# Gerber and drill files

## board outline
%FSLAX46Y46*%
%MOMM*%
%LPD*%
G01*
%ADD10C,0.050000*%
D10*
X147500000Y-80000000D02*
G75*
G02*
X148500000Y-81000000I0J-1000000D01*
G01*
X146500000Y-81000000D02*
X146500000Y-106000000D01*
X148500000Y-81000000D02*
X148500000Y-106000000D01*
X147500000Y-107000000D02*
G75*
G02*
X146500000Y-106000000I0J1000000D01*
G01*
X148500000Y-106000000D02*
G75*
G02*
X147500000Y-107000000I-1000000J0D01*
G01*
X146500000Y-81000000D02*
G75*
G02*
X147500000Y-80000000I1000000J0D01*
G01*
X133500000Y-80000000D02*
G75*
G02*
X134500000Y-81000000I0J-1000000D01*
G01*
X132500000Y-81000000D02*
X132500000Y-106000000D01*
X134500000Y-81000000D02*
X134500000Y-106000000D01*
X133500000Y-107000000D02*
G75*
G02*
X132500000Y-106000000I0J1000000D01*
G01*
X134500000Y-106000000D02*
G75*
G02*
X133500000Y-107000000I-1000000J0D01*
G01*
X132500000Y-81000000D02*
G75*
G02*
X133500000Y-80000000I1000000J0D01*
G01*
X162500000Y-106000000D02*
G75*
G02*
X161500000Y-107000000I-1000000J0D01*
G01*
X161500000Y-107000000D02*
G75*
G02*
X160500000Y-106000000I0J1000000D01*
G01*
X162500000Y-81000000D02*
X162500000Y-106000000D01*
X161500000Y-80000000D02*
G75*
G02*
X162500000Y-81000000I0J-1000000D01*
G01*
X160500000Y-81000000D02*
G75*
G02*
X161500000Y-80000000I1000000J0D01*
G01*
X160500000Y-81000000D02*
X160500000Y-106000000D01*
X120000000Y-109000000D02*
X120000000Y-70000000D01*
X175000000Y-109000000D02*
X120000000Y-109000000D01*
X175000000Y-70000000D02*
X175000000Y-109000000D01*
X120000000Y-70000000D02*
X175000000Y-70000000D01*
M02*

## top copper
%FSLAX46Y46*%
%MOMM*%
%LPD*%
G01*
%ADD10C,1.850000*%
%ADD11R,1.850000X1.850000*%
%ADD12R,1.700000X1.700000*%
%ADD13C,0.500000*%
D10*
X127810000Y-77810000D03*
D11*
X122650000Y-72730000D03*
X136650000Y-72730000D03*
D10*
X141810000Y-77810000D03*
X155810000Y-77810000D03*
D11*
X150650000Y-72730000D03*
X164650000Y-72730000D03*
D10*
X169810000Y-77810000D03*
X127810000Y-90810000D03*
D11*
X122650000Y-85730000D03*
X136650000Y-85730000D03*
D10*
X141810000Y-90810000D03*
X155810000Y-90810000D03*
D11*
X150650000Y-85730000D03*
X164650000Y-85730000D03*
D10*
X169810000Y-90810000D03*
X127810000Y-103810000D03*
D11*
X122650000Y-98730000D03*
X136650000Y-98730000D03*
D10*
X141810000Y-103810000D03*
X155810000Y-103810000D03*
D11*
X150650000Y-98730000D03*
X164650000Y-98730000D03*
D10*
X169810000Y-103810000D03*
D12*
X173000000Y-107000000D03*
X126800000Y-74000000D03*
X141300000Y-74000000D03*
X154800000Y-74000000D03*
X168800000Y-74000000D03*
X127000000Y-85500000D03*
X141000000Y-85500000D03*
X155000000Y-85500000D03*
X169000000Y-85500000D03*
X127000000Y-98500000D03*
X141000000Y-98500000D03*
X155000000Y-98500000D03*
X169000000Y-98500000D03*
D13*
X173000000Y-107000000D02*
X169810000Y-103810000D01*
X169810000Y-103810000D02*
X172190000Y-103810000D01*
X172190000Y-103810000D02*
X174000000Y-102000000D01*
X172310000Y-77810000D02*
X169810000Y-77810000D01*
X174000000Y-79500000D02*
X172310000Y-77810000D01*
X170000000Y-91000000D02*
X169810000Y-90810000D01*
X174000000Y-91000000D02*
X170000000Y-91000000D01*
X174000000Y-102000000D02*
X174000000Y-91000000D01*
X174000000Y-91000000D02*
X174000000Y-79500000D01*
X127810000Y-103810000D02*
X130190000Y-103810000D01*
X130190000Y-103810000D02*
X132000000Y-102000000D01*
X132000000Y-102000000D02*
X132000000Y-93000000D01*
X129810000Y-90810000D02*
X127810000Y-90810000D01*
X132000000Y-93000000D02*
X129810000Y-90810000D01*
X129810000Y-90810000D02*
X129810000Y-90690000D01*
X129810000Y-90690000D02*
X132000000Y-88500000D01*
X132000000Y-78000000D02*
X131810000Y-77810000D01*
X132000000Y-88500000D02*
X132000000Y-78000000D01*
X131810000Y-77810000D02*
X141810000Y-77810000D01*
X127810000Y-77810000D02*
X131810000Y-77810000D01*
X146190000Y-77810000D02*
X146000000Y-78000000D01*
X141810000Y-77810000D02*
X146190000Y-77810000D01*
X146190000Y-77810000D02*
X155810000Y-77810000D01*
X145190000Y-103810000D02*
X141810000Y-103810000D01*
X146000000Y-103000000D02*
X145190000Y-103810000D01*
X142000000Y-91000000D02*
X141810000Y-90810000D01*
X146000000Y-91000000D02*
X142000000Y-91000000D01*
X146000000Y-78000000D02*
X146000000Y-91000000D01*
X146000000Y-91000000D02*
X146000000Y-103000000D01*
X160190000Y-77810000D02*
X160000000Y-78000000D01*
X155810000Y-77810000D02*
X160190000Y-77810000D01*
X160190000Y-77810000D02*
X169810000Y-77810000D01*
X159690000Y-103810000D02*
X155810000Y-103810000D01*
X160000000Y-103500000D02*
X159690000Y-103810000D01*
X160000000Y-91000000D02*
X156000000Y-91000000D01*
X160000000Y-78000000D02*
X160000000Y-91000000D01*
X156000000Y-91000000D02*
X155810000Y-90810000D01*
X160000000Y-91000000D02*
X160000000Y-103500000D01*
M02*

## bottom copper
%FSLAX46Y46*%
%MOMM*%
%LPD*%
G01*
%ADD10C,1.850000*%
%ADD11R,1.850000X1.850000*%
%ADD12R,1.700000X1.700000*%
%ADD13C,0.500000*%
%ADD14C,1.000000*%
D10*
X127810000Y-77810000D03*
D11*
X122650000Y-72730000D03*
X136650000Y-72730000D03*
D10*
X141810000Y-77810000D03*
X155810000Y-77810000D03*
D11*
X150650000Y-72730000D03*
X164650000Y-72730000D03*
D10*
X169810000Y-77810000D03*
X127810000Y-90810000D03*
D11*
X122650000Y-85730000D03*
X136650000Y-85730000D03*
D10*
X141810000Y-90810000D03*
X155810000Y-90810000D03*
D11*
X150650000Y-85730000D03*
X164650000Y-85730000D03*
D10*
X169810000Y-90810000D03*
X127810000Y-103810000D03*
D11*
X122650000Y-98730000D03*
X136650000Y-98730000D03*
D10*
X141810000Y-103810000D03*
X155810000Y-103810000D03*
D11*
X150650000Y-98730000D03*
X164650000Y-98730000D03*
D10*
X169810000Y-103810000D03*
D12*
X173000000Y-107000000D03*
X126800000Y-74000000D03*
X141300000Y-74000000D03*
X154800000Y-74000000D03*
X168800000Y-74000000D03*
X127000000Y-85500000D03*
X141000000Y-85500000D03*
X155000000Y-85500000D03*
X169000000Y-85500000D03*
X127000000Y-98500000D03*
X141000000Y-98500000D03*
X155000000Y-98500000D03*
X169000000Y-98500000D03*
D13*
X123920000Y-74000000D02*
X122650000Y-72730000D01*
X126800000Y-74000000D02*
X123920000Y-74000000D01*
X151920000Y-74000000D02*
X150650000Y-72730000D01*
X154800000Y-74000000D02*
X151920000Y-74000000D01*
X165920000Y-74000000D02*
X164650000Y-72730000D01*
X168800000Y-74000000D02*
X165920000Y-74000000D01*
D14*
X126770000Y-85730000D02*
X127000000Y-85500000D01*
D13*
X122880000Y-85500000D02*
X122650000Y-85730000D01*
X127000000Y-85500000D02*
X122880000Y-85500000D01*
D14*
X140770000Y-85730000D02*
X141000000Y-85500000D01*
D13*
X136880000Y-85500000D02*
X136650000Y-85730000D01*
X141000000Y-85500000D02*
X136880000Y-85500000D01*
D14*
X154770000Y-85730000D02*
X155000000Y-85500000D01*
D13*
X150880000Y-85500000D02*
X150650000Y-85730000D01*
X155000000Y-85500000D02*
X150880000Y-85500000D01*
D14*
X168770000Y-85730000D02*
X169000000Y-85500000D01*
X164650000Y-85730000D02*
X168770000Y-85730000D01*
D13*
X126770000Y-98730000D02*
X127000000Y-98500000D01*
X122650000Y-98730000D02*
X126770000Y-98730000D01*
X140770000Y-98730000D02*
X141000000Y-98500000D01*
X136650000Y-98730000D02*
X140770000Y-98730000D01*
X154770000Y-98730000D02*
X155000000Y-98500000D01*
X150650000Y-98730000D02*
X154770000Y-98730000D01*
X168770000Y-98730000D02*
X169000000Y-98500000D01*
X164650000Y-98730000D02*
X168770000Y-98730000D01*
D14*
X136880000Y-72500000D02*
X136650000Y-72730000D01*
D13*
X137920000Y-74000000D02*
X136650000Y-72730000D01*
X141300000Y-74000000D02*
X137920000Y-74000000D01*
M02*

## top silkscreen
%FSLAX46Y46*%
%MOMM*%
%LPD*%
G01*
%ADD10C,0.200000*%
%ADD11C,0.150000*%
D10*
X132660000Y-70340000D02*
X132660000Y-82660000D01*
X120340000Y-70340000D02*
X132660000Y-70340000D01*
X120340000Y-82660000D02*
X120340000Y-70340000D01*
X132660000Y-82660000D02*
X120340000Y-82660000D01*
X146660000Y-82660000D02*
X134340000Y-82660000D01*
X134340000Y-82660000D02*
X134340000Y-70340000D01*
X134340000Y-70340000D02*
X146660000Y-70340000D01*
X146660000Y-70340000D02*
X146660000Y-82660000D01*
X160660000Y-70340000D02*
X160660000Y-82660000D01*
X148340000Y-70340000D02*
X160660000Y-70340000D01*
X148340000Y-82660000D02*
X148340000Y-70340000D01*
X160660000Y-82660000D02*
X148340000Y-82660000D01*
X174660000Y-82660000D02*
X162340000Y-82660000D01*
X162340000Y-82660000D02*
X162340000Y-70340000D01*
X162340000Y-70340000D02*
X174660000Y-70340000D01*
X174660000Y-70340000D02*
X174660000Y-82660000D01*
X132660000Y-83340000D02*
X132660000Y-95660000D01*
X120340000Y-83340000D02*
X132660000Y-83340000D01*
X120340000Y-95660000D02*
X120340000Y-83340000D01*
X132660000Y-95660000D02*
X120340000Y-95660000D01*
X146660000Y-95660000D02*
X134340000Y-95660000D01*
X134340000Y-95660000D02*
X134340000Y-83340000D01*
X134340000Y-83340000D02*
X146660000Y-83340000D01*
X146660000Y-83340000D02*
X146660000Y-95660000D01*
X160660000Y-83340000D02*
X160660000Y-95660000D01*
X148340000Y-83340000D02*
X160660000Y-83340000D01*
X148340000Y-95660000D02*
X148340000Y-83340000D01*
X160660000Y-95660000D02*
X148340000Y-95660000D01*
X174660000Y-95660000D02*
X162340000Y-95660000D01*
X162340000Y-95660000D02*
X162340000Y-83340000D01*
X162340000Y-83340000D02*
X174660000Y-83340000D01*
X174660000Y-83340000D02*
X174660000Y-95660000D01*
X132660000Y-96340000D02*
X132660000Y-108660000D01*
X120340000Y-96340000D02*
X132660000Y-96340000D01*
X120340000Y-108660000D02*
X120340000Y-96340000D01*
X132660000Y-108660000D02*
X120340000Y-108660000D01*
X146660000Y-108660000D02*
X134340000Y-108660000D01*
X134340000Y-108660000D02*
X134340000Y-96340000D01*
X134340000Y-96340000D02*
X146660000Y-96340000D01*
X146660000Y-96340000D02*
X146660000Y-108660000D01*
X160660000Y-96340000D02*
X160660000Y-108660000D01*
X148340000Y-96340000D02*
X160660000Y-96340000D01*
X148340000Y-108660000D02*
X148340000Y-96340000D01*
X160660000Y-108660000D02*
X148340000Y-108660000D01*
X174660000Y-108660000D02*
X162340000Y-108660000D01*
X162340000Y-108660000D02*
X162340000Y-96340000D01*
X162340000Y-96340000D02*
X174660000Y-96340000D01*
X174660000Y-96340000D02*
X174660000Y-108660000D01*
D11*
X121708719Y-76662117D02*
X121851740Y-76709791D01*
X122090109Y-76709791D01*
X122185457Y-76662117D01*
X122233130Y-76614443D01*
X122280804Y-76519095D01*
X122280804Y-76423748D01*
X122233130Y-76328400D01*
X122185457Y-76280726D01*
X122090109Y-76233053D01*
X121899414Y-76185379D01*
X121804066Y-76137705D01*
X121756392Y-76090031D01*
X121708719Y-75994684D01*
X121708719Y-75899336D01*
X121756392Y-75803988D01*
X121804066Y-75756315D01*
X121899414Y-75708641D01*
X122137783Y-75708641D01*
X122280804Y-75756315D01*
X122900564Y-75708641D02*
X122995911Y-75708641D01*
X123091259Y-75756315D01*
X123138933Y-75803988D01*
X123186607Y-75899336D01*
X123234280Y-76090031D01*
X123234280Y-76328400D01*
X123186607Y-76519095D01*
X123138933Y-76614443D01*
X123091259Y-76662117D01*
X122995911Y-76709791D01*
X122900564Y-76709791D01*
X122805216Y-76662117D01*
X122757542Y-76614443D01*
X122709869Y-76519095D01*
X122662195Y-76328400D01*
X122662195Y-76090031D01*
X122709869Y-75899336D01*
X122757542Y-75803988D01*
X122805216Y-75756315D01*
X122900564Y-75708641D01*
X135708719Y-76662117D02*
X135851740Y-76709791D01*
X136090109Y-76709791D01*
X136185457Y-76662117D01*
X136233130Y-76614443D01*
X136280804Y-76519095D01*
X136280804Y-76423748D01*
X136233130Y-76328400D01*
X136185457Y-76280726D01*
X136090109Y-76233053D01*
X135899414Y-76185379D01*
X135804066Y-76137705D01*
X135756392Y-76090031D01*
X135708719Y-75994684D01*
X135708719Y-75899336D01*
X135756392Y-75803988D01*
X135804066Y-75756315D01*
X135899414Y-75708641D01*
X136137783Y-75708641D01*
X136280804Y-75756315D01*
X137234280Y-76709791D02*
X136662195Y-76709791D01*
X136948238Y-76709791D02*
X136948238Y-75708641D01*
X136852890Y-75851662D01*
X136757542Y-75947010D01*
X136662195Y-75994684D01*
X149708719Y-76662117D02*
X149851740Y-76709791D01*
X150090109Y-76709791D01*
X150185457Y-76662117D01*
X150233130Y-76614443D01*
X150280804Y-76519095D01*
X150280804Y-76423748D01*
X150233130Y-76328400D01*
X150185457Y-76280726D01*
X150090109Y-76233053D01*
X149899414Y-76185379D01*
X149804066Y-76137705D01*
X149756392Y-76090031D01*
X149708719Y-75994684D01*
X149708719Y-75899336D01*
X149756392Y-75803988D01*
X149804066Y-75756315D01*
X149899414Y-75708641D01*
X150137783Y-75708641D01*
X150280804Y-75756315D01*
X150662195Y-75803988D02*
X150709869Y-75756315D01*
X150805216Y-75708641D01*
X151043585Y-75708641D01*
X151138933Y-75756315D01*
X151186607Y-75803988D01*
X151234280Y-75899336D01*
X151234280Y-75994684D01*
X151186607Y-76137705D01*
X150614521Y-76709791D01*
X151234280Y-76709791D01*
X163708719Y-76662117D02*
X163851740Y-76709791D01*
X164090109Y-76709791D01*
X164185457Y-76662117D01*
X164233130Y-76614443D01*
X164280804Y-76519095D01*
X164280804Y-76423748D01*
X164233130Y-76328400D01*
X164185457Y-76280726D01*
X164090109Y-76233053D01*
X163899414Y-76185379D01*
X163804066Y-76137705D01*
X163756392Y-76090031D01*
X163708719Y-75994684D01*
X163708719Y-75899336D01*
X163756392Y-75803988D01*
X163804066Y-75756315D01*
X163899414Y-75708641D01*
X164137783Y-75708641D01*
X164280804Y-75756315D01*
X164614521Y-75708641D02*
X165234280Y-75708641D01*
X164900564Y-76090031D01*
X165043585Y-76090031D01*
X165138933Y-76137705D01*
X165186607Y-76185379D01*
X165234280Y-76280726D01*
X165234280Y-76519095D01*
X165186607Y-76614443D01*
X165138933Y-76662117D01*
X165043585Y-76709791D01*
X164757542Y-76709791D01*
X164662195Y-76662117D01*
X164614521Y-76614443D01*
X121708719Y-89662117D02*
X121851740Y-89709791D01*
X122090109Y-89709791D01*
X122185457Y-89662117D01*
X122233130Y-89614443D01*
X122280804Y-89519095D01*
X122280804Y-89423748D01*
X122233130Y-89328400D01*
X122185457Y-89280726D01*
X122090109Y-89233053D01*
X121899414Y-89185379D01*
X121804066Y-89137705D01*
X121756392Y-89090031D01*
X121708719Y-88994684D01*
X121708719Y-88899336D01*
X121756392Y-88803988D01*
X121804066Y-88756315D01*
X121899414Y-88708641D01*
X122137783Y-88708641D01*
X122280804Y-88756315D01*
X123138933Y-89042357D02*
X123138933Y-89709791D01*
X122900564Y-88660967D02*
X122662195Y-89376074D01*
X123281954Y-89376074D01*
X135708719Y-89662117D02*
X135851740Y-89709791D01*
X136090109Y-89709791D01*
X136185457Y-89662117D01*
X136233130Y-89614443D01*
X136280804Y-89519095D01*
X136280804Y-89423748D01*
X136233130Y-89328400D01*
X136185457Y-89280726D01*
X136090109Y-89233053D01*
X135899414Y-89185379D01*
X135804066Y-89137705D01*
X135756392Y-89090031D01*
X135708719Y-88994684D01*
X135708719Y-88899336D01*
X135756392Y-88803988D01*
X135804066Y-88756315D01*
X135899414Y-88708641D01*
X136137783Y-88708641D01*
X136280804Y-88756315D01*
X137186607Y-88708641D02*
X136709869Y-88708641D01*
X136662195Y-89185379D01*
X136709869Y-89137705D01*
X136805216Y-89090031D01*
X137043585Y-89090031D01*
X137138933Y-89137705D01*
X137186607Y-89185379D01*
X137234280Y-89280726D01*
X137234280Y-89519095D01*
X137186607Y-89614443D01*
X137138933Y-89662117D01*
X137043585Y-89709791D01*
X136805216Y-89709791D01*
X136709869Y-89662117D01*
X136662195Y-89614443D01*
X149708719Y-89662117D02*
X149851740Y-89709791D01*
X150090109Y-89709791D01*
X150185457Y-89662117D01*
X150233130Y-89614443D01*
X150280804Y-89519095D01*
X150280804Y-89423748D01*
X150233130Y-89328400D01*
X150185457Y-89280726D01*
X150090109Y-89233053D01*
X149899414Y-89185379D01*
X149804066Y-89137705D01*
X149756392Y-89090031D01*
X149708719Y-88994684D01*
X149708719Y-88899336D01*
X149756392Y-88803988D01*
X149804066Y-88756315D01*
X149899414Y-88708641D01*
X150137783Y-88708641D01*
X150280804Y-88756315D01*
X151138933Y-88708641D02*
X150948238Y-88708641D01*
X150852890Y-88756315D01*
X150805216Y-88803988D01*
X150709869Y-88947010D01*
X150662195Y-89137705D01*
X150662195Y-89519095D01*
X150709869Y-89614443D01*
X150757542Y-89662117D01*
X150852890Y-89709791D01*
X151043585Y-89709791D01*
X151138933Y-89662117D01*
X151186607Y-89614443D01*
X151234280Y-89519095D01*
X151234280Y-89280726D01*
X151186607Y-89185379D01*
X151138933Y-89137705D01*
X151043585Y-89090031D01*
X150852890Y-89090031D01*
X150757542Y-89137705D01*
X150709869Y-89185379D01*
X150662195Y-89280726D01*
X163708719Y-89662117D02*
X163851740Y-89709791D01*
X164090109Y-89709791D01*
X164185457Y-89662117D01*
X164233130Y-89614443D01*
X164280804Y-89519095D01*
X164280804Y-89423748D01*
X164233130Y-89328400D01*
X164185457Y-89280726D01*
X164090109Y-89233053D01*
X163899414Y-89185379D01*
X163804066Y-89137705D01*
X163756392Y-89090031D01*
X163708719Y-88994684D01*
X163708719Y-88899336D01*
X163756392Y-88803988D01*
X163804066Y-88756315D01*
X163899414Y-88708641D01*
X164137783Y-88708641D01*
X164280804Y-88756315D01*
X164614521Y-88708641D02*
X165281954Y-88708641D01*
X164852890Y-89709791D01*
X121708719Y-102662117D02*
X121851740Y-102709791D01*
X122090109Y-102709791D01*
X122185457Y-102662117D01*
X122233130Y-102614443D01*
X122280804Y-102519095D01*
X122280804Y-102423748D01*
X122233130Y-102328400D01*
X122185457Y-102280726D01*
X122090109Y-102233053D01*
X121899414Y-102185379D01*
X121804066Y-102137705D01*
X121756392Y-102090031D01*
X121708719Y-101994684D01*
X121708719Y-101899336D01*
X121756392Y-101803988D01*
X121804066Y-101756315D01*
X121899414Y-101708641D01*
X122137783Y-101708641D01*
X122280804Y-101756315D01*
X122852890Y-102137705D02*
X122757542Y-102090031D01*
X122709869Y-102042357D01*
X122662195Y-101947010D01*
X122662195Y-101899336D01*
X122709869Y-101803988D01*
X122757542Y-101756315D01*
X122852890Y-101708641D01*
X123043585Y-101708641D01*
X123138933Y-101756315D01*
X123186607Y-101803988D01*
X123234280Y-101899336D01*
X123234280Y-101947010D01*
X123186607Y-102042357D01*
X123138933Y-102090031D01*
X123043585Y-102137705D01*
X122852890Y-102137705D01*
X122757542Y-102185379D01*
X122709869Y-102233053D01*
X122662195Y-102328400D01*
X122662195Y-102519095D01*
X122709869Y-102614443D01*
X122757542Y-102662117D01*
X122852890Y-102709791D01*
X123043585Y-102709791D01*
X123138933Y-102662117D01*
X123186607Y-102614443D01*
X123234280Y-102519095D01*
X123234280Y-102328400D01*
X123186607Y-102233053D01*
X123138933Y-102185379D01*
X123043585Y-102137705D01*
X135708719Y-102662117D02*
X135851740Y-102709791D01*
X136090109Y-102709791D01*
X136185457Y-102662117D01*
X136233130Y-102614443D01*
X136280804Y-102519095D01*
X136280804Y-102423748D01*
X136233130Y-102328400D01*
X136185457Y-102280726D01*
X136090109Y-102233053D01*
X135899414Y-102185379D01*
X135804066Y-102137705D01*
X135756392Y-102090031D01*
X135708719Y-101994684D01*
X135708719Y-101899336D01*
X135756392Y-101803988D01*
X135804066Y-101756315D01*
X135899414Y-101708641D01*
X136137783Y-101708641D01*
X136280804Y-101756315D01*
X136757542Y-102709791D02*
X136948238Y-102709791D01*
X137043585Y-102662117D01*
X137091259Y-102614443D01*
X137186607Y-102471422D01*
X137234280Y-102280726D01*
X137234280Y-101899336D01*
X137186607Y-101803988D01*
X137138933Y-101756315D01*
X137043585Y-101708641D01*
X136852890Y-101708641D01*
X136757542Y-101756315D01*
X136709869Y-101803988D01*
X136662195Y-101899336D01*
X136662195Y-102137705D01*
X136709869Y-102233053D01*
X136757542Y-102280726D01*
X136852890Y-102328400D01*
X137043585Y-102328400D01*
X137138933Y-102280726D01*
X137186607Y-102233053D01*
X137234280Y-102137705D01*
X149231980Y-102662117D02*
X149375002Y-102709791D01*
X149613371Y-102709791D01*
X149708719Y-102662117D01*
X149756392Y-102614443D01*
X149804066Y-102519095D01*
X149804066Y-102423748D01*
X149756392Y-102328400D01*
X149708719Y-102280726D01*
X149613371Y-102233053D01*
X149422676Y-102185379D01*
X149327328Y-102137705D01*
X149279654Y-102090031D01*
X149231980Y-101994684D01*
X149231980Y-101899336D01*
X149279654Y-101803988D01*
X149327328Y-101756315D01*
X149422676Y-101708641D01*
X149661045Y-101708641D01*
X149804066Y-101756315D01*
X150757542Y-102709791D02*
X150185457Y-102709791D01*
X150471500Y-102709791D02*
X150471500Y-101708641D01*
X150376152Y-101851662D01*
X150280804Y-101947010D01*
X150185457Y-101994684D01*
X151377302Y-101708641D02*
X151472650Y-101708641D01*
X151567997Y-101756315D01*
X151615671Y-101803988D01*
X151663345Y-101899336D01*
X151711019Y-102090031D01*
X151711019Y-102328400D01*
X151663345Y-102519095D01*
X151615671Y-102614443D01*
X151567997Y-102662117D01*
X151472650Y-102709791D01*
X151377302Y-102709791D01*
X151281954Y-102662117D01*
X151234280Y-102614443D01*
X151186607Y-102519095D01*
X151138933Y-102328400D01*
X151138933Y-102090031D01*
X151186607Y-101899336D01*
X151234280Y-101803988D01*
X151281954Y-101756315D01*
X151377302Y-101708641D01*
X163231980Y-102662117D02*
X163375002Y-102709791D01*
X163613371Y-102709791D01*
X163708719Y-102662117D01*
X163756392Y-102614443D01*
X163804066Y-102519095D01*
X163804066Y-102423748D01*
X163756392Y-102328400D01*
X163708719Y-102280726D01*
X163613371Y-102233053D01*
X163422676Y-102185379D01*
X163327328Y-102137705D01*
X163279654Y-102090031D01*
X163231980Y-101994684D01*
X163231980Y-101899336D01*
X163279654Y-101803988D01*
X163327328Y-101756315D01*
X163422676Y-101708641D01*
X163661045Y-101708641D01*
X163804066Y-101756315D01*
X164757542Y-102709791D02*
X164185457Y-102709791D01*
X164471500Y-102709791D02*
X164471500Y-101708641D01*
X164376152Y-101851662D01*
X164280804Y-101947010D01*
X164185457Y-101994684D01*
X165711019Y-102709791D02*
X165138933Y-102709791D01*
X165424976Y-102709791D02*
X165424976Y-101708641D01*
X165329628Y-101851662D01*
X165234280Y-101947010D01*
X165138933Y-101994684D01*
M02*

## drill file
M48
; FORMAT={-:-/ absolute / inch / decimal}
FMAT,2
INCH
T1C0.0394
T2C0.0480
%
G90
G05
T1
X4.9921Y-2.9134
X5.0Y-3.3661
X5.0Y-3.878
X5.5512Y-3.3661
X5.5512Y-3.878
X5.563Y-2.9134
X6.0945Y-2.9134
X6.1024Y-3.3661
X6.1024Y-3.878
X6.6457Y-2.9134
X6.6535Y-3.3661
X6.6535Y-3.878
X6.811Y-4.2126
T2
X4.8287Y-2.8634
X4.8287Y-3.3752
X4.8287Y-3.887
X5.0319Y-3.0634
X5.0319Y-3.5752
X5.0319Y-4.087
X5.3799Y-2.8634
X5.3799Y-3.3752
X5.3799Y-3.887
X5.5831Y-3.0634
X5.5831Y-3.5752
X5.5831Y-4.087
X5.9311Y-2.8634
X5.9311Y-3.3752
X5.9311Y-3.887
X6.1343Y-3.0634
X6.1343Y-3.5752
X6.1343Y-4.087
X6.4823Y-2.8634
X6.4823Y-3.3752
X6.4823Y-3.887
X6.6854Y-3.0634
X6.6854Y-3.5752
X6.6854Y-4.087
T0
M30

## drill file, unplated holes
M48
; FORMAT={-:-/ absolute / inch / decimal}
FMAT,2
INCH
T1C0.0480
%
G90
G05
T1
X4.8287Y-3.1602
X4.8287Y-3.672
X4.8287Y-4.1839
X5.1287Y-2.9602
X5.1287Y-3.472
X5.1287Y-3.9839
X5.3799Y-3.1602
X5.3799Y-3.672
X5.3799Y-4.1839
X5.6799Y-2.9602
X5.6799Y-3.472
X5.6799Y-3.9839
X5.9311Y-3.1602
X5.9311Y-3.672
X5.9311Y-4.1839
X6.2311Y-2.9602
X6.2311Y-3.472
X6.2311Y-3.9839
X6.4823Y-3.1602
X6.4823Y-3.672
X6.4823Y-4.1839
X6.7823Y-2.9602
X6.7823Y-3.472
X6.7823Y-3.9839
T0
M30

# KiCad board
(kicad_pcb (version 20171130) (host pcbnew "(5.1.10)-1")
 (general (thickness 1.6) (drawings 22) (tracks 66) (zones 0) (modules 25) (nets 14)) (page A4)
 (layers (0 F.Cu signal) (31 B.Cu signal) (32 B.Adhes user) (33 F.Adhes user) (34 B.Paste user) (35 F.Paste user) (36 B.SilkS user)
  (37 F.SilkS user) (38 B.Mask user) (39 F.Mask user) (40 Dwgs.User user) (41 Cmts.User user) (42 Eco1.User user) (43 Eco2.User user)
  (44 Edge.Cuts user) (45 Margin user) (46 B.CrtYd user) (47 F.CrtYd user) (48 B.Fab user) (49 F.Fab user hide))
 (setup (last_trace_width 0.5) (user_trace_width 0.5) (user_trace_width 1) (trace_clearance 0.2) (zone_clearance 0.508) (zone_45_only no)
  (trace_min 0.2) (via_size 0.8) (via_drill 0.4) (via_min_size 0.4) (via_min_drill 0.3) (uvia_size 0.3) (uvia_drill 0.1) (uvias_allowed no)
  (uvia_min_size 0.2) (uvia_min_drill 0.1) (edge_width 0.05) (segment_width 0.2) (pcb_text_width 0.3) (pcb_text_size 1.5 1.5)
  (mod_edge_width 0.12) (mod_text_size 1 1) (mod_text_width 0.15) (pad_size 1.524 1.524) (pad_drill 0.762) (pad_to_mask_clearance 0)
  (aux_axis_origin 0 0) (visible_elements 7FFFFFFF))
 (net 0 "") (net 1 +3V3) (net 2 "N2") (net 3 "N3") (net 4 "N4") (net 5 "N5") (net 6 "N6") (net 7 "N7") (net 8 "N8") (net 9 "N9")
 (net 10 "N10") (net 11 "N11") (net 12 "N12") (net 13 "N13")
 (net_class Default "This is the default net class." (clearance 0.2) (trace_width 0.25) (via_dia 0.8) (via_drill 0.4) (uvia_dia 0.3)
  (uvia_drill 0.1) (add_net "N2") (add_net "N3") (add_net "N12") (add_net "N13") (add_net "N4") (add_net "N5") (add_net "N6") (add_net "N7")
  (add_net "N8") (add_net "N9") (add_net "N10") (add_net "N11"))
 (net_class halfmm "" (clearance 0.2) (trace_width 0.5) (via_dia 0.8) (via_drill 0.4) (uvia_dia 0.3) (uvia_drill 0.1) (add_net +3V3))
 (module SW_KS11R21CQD (layer F.Cu) (at 126.5 76.5)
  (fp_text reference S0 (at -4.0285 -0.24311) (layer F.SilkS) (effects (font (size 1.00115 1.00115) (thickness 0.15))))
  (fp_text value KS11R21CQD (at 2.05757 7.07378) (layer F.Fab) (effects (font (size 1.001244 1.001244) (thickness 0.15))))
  (fp_line (start 6.16 -6.16) (end 6.16 6.16) (layer F.SilkS) (width 0.2))
  (fp_line (start -6.16 -6.16) (end 6.16 -6.16) (layer F.SilkS) (width 0.2))
  (fp_line (start -6.16 6.16) (end -6.16 -6.16) (layer F.SilkS) (width 0.2))
  (fp_line (start 6.16 6.16) (end -6.16 6.16) (layer F.SilkS) (width 0.2))
  (pad None np_thru_hole circle (at -3.85 3.77) (size 1.22 1.22) (drill 1.22) (layers *.Cu *.Mask))
  (pad None np_thru_hole circle (at 3.77 -1.31) (size 1.22 1.22) (drill 1.22) (layers *.Cu *.Mask))
  (pad 3 thru_hole circle (at 1.31 1.31) (size 1.85 1.85) (drill 1.22) (layers *.Cu *.Mask) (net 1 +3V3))
  (pad 1 thru_hole rect (at -3.85 -3.77) (size 1.85 1.85) (drill 1.22) (layers *.Cu *.Mask) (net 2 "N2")))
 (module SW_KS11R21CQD (layer F.Cu) (at 140.5 76.5)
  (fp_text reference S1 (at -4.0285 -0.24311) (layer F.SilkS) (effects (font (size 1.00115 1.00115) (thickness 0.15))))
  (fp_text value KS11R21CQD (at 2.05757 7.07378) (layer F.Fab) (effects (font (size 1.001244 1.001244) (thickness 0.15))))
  (fp_line (start 6.16 6.16) (end -6.16 6.16) (layer F.SilkS) (width 0.2))
  (fp_line (start -6.16 6.16) (end -6.16 -6.16) (layer F.SilkS) (width 0.2))
  (fp_line (start -6.16 -6.16) (end 6.16 -6.16) (layer F.SilkS) (width 0.2))
  (fp_line (start 6.16 -6.16) (end 6.16 6.16) (layer F.SilkS) (width 0.2))
  (pad 1 thru_hole rect (at -3.85 -3.77) (size 1.85 1.85) (drill 1.22) (layers *.Cu *.Mask) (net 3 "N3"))
  (pad 3 thru_hole circle (at 1.31 1.31) (size 1.85 1.85) (drill 1.22) (layers *.Cu *.Mask) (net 1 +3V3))
  (pad None np_thru_hole circle (at 3.77 -1.31) (size 1.22 1.22) (drill 1.22) (layers *.Cu *.Mask))
  (pad None np_thru_hole circle (at -3.85 3.77) (size 1.22 1.22) (drill 1.22) (layers *.Cu *.Mask)))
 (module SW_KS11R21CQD (layer F.Cu) (at 154.5 76.5)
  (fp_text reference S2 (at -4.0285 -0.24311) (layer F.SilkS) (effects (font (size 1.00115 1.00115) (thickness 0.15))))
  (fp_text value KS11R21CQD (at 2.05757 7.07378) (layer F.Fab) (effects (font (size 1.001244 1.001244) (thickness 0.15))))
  (fp_line (start 6.16 -6.16) (end 6.16 6.16) (layer F.SilkS) (width 0.2))
  (fp_line (start -6.16 -6.16) (end 6.16 -6.16) (layer F.SilkS) (width 0.2))
  (fp_line (start -6.16 6.16) (end -6.16 -6.16) (layer F.SilkS) (width 0.2))
  (fp_line (start 6.16 6.16) (end -6.16 6.16) (layer F.SilkS) (width 0.2))
  (pad None np_thru_hole circle (at -3.85 3.77) (size 1.22 1.22) (drill 1.22) (layers *.Cu *.Mask))
  (pad None np_thru_hole circle (at 3.77 -1.31) (size 1.22 1.22) (drill 1.22) (layers *.Cu *.Mask))
  (pad 3 thru_hole circle (at 1.31 1.31) (size 1.85 1.85) (drill 1.22) (layers *.Cu *.Mask) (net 1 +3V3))
  (pad 1 thru_hole rect (at -3.85 -3.77) (size 1.85 1.85) (drill 1.22) (layers *.Cu *.Mask) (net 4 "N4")))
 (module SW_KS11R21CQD (layer F.Cu) (at 168.5 76.5)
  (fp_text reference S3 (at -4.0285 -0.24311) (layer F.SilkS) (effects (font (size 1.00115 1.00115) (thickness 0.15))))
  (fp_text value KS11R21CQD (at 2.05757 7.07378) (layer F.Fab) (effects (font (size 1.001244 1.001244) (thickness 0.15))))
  (fp_line (start 6.16 6.16) (end -6.16 6.16) (layer F.SilkS) (width 0.2))
  (fp_line (start -6.16 6.16) (end -6.16 -6.16) (layer F.SilkS) (width 0.2))
  (fp_line (start -6.16 -6.16) (end 6.16 -6.16) (layer F.SilkS) (width 0.2))
  (fp_line (start 6.16 -6.16) (end 6.16 6.16) (layer F.SilkS) (width 0.2))
  (pad 1 thru_hole rect (at -3.85 -3.77) (size 1.85 1.85) (drill 1.22) (layers *.Cu *.Mask) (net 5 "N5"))
  (pad 3 thru_hole circle (at 1.31 1.31) (size 1.85 1.85) (drill 1.22) (layers *.Cu *.Mask) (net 1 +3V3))
  (pad None np_thru_hole circle (at 3.77 -1.31) (size 1.22 1.22) (drill 1.22) (layers *.Cu *.Mask))
  (pad None np_thru_hole circle (at -3.85 3.77) (size 1.22 1.22) (drill 1.22) (layers *.Cu *.Mask)))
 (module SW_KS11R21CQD (layer F.Cu) (at 126.5 89.5)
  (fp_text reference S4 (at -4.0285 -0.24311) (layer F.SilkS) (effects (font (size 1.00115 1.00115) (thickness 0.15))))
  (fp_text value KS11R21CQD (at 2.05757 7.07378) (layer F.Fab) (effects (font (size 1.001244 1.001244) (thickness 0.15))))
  (fp_line (start 6.16 -6.16) (end 6.16 6.16) (layer F.SilkS) (width 0.2))
  (fp_line (start -6.16 -6.16) (end 6.16 -6.16) (layer F.SilkS) (width 0.2))
  (fp_line (start -6.16 6.16) (end -6.16 -6.16) (layer F.SilkS) (width 0.2))
  (fp_line (start 6.16 6.16) (end -6.16 6.16) (layer F.SilkS) (width 0.2))
  (pad None np_thru_hole circle (at -3.85 3.77) (size 1.22 1.22) (drill 1.22) (layers *.Cu *.Mask))
  (pad None np_thru_hole circle (at 3.77 -1.31) (size 1.22 1.22) (drill 1.22) (layers *.Cu *.Mask))
  (pad 3 thru_hole circle (at 1.31 1.31) (size 1.85 1.85) (drill 1.22) (layers *.Cu *.Mask) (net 1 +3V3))
  (pad 1 thru_hole rect (at -3.85 -3.77) (size 1.85 1.85) (drill 1.22) (layers *.Cu *.Mask) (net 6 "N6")))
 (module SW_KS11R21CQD (layer F.Cu) (at 140.5 89.5)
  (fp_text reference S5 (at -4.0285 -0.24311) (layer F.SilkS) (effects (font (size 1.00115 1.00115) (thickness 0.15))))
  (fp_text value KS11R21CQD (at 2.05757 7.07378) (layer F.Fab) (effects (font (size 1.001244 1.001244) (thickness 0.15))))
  (fp_line (start 6.16 6.16) (end -6.16 6.16) (layer F.SilkS) (width 0.2))
  (fp_line (start -6.16 6.16) (end -6.16 -6.16) (layer F.SilkS) (width 0.2))
  (fp_line (start -6.16 -6.16) (end 6.16 -6.16) (layer F.SilkS) (width 0.2))
  (fp_line (start 6.16 -6.16) (end 6.16 6.16) (layer F.SilkS) (width 0.2))
  (pad 1 thru_hole rect (at -3.85 -3.77) (size 1.85 1.85) (drill 1.22) (layers *.Cu *.Mask) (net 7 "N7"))
  (pad 3 thru_hole circle (at 1.31 1.31) (size 1.85 1.85) (drill 1.22) (layers *.Cu *.Mask) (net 1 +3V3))
  (pad None np_thru_hole circle (at 3.77 -1.31) (size 1.22 1.22) (drill 1.22) (layers *.Cu *.Mask))
  (pad None np_thru_hole circle (at -3.85 3.77) (size 1.22 1.22) (drill 1.22) (layers *.Cu *.Mask)))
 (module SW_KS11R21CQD (layer F.Cu) (at 154.5 89.5)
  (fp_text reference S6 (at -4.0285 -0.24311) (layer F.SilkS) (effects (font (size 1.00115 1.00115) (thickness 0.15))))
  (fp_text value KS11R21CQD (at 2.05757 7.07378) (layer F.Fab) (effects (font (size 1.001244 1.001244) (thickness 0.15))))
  (fp_line (start 6.16 -6.16) (end 6.16 6.16) (layer F.SilkS) (width 0.2))
  (fp_line (start -6.16 -6.16) (end 6.16 -6.16) (layer F.SilkS) (width 0.2))
  (fp_line (start -6.16 6.16) (end -6.16 -6.16) (layer F.SilkS) (width 0.2))
  (fp_line (start 6.16 6.16) (end -6.16 6.16) (layer F.SilkS) (width 0.2))
  (pad None np_thru_hole circle (at -3.85 3.77) (size 1.22 1.22) (drill 1.22) (layers *.Cu *.Mask))
  (pad None np_thru_hole circle (at 3.77 -1.31) (size 1.22 1.22) (drill 1.22) (layers *.Cu *.Mask))
  (pad 3 thru_hole circle (at 1.31 1.31) (size 1.85 1.85) (drill 1.22) (layers *.Cu *.Mask) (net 1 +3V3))
  (pad 1 thru_hole rect (at -3.85 -3.77) (size 1.85 1.85) (drill 1.22) (layers *.Cu *.Mask) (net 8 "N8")))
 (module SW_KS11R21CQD (layer F.Cu) (at 168.5 89.5)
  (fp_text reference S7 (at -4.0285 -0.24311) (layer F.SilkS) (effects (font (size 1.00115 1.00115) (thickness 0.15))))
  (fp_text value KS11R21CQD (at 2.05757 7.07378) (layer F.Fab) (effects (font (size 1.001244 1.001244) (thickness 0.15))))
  (fp_line (start 6.16 6.16) (end -6.16 6.16) (layer F.SilkS) (width 0.2))
  (fp_line (start -6.16 6.16) (end -6.16 -6.16) (layer F.SilkS) (width 0.2))
  (fp_line (start -6.16 -6.16) (end 6.16 -6.16) (layer F.SilkS) (width 0.2))
  (fp_line (start 6.16 -6.16) (end 6.16 6.16) (layer F.SilkS) (width 0.2))
  (pad 1 thru_hole rect (at -3.85 -3.77) (size 1.85 1.85) (drill 1.22) (layers *.Cu *.Mask) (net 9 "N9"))
  (pad 3 thru_hole circle (at 1.31 1.31) (size 1.85 1.85) (drill 1.22) (layers *.Cu *.Mask) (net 1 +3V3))
  (pad None np_thru_hole circle (at 3.77 -1.31) (size 1.22 1.22) (drill 1.22) (layers *.Cu *.Mask))
  (pad None np_thru_hole circle (at -3.85 3.77) (size 1.22 1.22) (drill 1.22) (layers *.Cu *.Mask)))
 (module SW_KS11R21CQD (layer F.Cu) (at 126.5 102.5)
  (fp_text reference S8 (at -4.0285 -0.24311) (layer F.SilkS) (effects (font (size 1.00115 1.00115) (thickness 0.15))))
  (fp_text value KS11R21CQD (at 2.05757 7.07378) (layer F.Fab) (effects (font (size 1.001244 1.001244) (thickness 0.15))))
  (fp_line (start 6.16 -6.16) (end 6.16 6.16) (layer F.SilkS) (width 0.2))
  (fp_line (start -6.16 -6.16) (end 6.16 -6.16) (layer F.SilkS) (width 0.2))
  (fp_line (start -6.16 6.16) (end -6.16 -6.16) (layer F.SilkS) (width 0.2))
  (fp_line (start 6.16 6.16) (end -6.16 6.16) (layer F.SilkS) (width 0.2))
  (pad None np_thru_hole circle (at -3.85 3.77) (size 1.22 1.22) (drill 1.22) (layers *.Cu *.Mask))
  (pad None np_thru_hole circle (at 3.77 -1.31) (size 1.22 1.22) (drill 1.22) (layers *.Cu *.Mask))
  (pad 3 thru_hole circle (at 1.31 1.31) (size 1.85 1.85) (drill 1.22) (layers *.Cu *.Mask) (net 1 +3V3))
  (pad 1 thru_hole rect (at -3.85 -3.77) (size 1.85 1.85) (drill 1.22) (layers *.Cu *.Mask) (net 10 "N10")))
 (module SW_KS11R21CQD (layer F.Cu) (at 140.5 102.5)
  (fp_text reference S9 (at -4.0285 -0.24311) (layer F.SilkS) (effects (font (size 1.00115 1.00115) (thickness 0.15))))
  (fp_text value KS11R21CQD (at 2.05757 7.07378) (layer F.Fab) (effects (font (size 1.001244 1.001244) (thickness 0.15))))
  (fp_line (start 6.16 6.16) (end -6.16 6.16) (layer F.SilkS) (width 0.2))
  (fp_line (start -6.16 6.16) (end -6.16 -6.16) (layer F.SilkS) (width 0.2))
  (fp_line (start -6.16 -6.16) (end 6.16 -6.16) (layer F.SilkS) (width 0.2))
  (fp_line (start 6.16 -6.16) (end 6.16 6.16) (layer F.SilkS) (width 0.2))
  (pad 1 thru_hole rect (at -3.85 -3.77) (size 1.85 1.85) (drill 1.22) (layers *.Cu *.Mask) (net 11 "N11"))
  (pad 3 thru_hole circle (at 1.31 1.31) (size 1.85 1.85) (drill 1.22) (layers *.Cu *.Mask) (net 1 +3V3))
  (pad None np_thru_hole circle (at 3.77 -1.31) (size 1.22 1.22) (drill 1.22) (layers *.Cu *.Mask))
  (pad None np_thru_hole circle (at -3.85 3.77) (size 1.22 1.22) (drill 1.22) (layers *.Cu *.Mask)))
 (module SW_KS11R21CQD (layer F.Cu) (at 154.5 102.5)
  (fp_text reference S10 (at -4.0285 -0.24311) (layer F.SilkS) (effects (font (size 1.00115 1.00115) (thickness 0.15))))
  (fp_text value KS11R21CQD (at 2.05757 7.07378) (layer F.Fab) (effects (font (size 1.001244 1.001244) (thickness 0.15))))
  (fp_line (start 6.16 -6.16) (end 6.16 6.16) (layer F.SilkS) (width 0.2))
  (fp_line (start -6.16 -6.16) (end 6.16 -6.16) (layer F.SilkS) (width 0.2))
  (fp_line (start -6.16 6.16) (end -6.16 -6.16) (layer F.SilkS) (width 0.2))
  (fp_line (start 6.16 6.16) (end -6.16 6.16) (layer F.SilkS) (width 0.2))
  (pad None np_thru_hole circle (at -3.85 3.77) (size 1.22 1.22) (drill 1.22) (layers *.Cu *.Mask))
  (pad None np_thru_hole circle (at 3.77 -1.31) (size 1.22 1.22) (drill 1.22) (layers *.Cu *.Mask))
  (pad 3 thru_hole circle (at 1.31 1.31) (size 1.85 1.85) (drill 1.22) (layers *.Cu *.Mask) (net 1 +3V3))
  (pad 1 thru_hole rect (at -3.85 -3.77) (size 1.85 1.85) (drill 1.22) (layers *.Cu *.Mask) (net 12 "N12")))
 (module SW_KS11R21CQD (layer F.Cu) (at 168.5 102.5)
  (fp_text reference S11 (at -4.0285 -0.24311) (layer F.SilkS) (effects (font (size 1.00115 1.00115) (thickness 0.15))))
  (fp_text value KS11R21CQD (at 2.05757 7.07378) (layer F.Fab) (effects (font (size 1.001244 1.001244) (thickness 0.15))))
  (fp_line (start 6.16 6.16) (end -6.16 6.16) (layer F.SilkS) (width 0.2))
  (fp_line (start -6.16 6.16) (end -6.16 -6.16) (layer F.SilkS) (width 0.2))
  (fp_line (start -6.16 -6.16) (end 6.16 -6.16) (layer F.SilkS) (width 0.2))
  (fp_line (start 6.16 -6.16) (end 6.16 6.16) (layer F.SilkS) (width 0.2))
  (pad 1 thru_hole rect (at -3.85 -3.77) (size 1.85 1.85) (drill 1.22) (layers *.Cu *.Mask) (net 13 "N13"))
  (pad 3 thru_hole circle (at 1.31 1.31) (size 1.85 1.85) (drill 1.22) (layers *.Cu *.Mask) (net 1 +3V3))
  (pad None np_thru_hole circle (at 3.77 -1.31) (size 1.22 1.22) (drill 1.22) (layers *.Cu *.Mask))
  (pad None np_thru_hole circle (at -3.85 3.77) (size 1.22 1.22) (drill 1.22) (layers *.Cu *.Mask)))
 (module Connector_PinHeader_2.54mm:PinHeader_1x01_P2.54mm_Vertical (layer B.Cu) (at 173 107)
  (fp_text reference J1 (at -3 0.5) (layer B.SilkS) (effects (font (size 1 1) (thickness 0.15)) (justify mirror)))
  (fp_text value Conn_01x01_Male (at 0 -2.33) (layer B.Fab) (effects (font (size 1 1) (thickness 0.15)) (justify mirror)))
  (pad 1 thru_hole rect (at 0 0) (size 1.7 1.7) (drill 1) (layers *.Cu *.Mask) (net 1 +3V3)))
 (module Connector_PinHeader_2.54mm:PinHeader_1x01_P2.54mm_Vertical (layer B.Cu) (at 126.8 74)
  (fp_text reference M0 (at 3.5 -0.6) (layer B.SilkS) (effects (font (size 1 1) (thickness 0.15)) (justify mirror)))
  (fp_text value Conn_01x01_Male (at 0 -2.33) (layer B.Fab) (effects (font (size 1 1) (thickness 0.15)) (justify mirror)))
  (pad 1 thru_hole rect (at 0 0) (size 1.7 1.7) (drill 1) (layers *.Cu *.Mask) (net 2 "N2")))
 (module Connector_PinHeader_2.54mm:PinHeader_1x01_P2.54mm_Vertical (layer B.Cu) (at 141.3 74)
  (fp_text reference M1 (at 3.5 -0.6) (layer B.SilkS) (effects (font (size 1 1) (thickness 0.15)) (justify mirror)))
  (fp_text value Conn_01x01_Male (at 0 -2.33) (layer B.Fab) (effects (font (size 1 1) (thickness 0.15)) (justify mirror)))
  (pad 1 thru_hole rect (at 0 0) (size 1.7 1.7) (drill 1) (layers *.Cu *.Mask) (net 3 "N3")))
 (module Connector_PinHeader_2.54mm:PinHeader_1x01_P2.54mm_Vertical (layer B.Cu) (at 154.8 74)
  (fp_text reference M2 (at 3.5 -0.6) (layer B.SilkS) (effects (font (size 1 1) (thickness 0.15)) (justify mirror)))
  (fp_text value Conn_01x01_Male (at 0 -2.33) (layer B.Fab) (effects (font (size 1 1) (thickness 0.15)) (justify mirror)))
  (pad 1 thru_hole rect (at 0 0) (size 1.7 1.7) (drill 1) (layers *.Cu *.Mask) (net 4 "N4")))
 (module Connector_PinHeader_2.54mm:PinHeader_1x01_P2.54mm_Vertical (layer B.Cu) (at 168.8 74)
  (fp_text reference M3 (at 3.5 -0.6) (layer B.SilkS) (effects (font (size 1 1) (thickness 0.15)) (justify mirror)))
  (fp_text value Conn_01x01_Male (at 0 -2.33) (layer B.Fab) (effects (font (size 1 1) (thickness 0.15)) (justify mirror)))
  (pad 1 thru_hole rect (at 0 0) (size 1.7 1.7) (drill 1) (layers *.Cu *.Mask) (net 5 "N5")))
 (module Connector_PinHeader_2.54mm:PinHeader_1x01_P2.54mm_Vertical (layer B.Cu) (at 127 85.5)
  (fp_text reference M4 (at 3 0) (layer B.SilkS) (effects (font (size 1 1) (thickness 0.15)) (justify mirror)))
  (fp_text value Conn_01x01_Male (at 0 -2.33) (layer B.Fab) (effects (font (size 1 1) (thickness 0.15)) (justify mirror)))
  (pad 1 thru_hole rect (at 0 0) (size 1.7 1.7) (drill 1) (layers *.Cu *.Mask) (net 6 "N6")))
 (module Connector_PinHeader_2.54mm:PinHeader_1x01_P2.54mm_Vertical (layer B.Cu) (at 141 85.5)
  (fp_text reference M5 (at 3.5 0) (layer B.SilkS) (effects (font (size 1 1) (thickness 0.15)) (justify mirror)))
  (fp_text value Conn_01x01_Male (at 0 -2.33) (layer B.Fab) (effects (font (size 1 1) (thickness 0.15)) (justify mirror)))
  (pad 1 thru_hole rect (at 0 0) (size 1.7 1.7) (drill 1) (layers *.Cu *.Mask) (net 7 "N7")))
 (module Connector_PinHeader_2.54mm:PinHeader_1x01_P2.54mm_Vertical (layer B.Cu) (at 155 85.5)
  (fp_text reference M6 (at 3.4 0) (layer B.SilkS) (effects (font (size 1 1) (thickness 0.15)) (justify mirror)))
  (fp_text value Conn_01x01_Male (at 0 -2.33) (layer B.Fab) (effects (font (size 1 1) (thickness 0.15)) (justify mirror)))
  (pad 1 thru_hole rect (at 0 0) (size 1.7 1.7) (drill 1) (layers *.Cu *.Mask) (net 8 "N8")))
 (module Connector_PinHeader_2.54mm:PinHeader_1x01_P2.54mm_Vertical (layer B.Cu) (at 169 85.5)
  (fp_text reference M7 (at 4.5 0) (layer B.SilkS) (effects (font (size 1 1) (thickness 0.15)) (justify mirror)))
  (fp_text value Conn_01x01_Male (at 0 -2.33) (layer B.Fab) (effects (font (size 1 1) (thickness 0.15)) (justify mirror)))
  (pad 1 thru_hole rect (at 0 0) (size 1.7 1.7) (drill 1) (layers *.Cu *.Mask) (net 9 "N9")))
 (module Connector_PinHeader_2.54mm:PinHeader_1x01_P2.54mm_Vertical (layer B.Cu) (at 127 98.5)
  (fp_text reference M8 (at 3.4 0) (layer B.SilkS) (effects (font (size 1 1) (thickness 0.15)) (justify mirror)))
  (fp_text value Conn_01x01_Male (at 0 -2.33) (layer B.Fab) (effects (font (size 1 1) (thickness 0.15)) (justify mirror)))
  (pad 1 thru_hole rect (at 0 0) (size 1.7 1.7) (drill 1) (layers *.Cu *.Mask) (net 10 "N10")))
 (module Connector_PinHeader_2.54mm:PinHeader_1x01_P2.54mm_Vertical (layer B.Cu) (at 141 98.5)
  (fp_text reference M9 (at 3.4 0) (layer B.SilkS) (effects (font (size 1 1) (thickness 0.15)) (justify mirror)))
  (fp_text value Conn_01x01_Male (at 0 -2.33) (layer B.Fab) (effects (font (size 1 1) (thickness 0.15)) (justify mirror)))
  (pad 1 thru_hole rect (at 0 0) (size 1.7 1.7) (drill 1) (layers *.Cu *.Mask) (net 11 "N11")))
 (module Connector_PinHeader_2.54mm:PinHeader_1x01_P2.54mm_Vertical (layer B.Cu) (at 155 98.5)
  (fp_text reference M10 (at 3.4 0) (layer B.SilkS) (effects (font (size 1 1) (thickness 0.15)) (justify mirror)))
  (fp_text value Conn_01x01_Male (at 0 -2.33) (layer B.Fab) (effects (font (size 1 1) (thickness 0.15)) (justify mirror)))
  (pad 1 thru_hole rect (at 0 0) (size 1.7 1.7) (drill 1) (layers *.Cu *.Mask) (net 12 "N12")))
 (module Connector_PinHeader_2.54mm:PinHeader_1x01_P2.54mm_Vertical (layer B.Cu) (at 169 98.5)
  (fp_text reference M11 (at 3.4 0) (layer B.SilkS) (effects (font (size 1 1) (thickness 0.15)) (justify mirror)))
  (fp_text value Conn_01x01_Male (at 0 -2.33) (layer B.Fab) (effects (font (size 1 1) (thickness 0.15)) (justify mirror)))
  (pad 1 thru_hole rect (at 0 0) (size 1.7 1.7) (drill 1) (layers *.Cu *.Mask) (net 13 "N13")))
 (gr_arc (start 147.5 81) (end 148.5 81) (angle -90) (layer Edge.Cuts) (width 0.05))
 (gr_line (start 146.5 81) (end 146.5 106) (layer Edge.Cuts) (width 0.05))
 (gr_line (start 148.5 81) (end 148.5 106) (layer Edge.Cuts) (width 0.05))
 (gr_arc (start 147.5 106) (end 146.5 106) (angle -90) (layer Edge.Cuts) (width 0.05))
 (gr_arc (start 147.5 106) (end 147.5 107) (angle -90) (layer Edge.Cuts) (width 0.05))
 (gr_arc (start 147.5 81) (end 147.5 80) (angle -90) (layer Edge.Cuts) (width 0.05))
 (gr_arc (start 133.5 81) (end 134.5 81) (angle -90) (layer Edge.Cuts) (width 0.05))
 (gr_line (start 132.5 81) (end 132.5 106) (layer Edge.Cuts) (width 0.05))
 (gr_line (start 134.5 81) (end 134.5 106) (layer Edge.Cuts) (width 0.05))
 (gr_arc (start 133.5 106) (end 132.5 106) (angle -90) (layer Edge.Cuts) (width 0.05))
 (gr_arc (start 133.5 106) (end 133.5 107) (angle -90) (layer Edge.Cuts) (width 0.05))
 (gr_arc (start 133.5 81) (end 133.5 80) (angle -90) (layer Edge.Cuts) (width 0.05))
 (gr_arc (start 161.5 106) (end 161.5 107) (angle -90) (layer Edge.Cuts) (width 0.05))
 (gr_arc (start 161.5 106) (end 160.5 106) (angle -90) (layer Edge.Cuts) (width 0.05))
 (gr_line (start 162.5 81) (end 162.5 106) (layer Edge.Cuts) (width 0.05))
 (gr_arc (start 161.5 81) (end 162.5 81) (angle -90) (layer Edge.Cuts) (width 0.05))
 (gr_arc (start 161.5 81) (end 161.5 80) (angle -90) (layer Edge.Cuts) (width 0.05))
 (gr_line (start 160.5 81) (end 160.5 106) (layer Edge.Cuts) (width 0.05))
 (gr_line (start 120 109) (end 120 70) (layer Edge.Cuts) (width 0.05))
 (gr_line (start 175 109) (end 120 109) (layer Edge.Cuts) (width 0.05))
 (gr_line (start 175 70) (end 175 109) (layer Edge.Cuts) (width 0.05))
 (gr_line (start 120 70) (end 175 70) (layer Edge.Cuts) (width 0.05))
 (segment (start 173 107) (end 169.81 103.81) (width 0.5) (layer F.Cu) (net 1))
 (segment (start 169.81 103.81) (end 172.19 103.81) (width 0.5) (layer F.Cu) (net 1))
 (segment (start 172.19 103.81) (end 174 102) (width 0.5) (layer F.Cu) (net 1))
 (segment (start 172.31 77.81) (end 169.81 77.81) (width 0.5) (layer F.Cu) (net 1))
 (segment (start 174 79.5) (end 172.31 77.81) (width 0.5) (layer F.Cu) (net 1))
 (segment (start 170 91) (end 169.81 90.81) (width 0.5) (layer F.Cu) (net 1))
 (segment (start 174 91) (end 170 91) (width 0.5) (layer F.Cu) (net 1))
 (segment (start 174 102) (end 174 91) (width 0.5) (layer F.Cu) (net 1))
 (segment (start 174 91) (end 174 79.5) (width 0.5) (layer F.Cu) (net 1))
 (segment (start 127.81 103.81) (end 130.19 103.81) (width 0.5) (layer F.Cu) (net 1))
 (segment (start 130.19 103.81) (end 132 102) (width 0.5) (layer F.Cu) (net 1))
 (segment (start 132 102) (end 132 93) (width 0.5) (layer F.Cu) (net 1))
 (segment (start 129.81 90.81) (end 127.81 90.81) (width 0.5) (layer F.Cu) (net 1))
 (segment (start 132 93) (end 129.81 90.81) (width 0.5) (layer F.Cu) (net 1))
 (segment (start 129.81 90.81) (end 129.81 90.69) (width 0.5) (layer F.Cu) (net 1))
 (segment (start 129.81 90.69) (end 132 88.5) (width 0.5) (layer F.Cu) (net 1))
 (segment (start 132 78) (end 131.81 77.81) (width 0.5) (layer F.Cu) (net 1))
 (segment (start 132 88.5) (end 132 78) (width 0.5) (layer F.Cu) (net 1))
 (segment (start 131.81 77.81) (end 141.81 77.81) (width 0.5) (layer F.Cu) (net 1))
 (segment (start 127.81 77.81) (end 131.81 77.81) (width 0.5) (layer F.Cu) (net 1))
 (segment (start 146.19 77.81) (end 146 78) (width 0.5) (layer F.Cu) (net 1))
 (segment (start 141.81 77.81) (end 146.19 77.81) (width 0.5) (layer F.Cu) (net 1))
 (segment (start 146.19 77.81) (end 155.81 77.81) (width 0.5) (layer F.Cu) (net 1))
 (segment (start 145.19 103.81) (end 141.81 103.81) (width 0.5) (layer F.Cu) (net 1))
 (segment (start 146 103) (end 145.19 103.81) (width 0.5) (layer F.Cu) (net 1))
 (segment (start 142 91) (end 141.81 90.81) (width 0.5) (layer F.Cu) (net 1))
 (segment (start 146 91) (end 142 91) (width 0.5) (layer F.Cu) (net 1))
 (segment (start 146 78) (end 146 91) (width 0.5) (layer F.Cu) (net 1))
 (segment (start 146 91) (end 146 103) (width 0.5) (layer F.Cu) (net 1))
 (segment (start 160.19 77.81) (end 160 78) (width 0.5) (layer F.Cu) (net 1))
 (segment (start 155.81 77.81) (end 160.19 77.81) (width 0.5) (layer F.Cu) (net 1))
 (segment (start 160.19 77.81) (end 169.81 77.81) (width 0.5) (layer F.Cu) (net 1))
 (segment (start 159.69 103.81) (end 155.81 103.81) (width 0.5) (layer F.Cu) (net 1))
 (segment (start 160 103.5) (end 159.69 103.81) (width 0.5) (layer F.Cu) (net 1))
 (segment (start 160 91) (end 156 91) (width 0.5) (layer F.Cu) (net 1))
 (segment (start 160 78) (end 160 91) (width 0.5) (layer F.Cu) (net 1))
 (segment (start 156 91) (end 155.81 90.81) (width 0.5) (layer F.Cu) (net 1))
 (segment (start 160 91) (end 160 103.5) (width 0.5) (layer F.Cu) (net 1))
 (segment (start 123.92 74) (end 122.65 72.73) (width 0.5) (layer B.Cu) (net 2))
 (segment (start 126.8 74) (end 123.92 74) (width 0.5) (layer B.Cu) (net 2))
 (segment (start 151.92 74) (end 150.65 72.73) (width 0.5) (layer B.Cu) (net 4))
 (segment (start 154.8 74) (end 151.92 74) (width 0.5) (layer B.Cu) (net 4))
 (segment (start 165.92 74) (end 164.65 72.73) (width 0.5) (layer B.Cu) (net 5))
 (segment (start 168.8 74) (end 165.92 74) (width 0.5) (layer B.Cu) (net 5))
 (segment (start 126.77 85.73) (end 127 85.5) (width 1) (layer B.Cu) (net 6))
 (segment (start 122.88 85.5) (end 122.65 85.73) (width 0.5) (layer B.Cu) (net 6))
 (segment (start 127 85.5) (end 122.88 85.5) (width 0.5) (layer B.Cu) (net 6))
 (segment (start 140.77 85.73) (end 141 85.5) (width 1) (layer B.Cu) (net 7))
 (segment (start 136.88 85.5) (end 136.65 85.73) (width 0.5) (layer B.Cu) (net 7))
 (segment (start 141 85.5) (end 136.88 85.5) (width 0.5) (layer B.Cu) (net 7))
 (segment (start 154.77 85.73) (end 155 85.5) (width 1) (layer B.Cu) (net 8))
 (segment (start 150.88 85.5) (end 150.65 85.73) (width 0.5) (layer B.Cu) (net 8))
 (segment (start 155 85.5) (end 150.88 85.5) (width 0.5) (layer B.Cu) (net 8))
 (segment (start 168.77 85.73) (end 169 85.5) (width 1) (layer B.Cu) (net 9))
 (segment (start 164.65 85.73) (end 168.77 85.73) (width 1) (layer B.Cu) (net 9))
 (segment (start 126.77 98.73) (end 127 98.5) (width 0.5) (layer B.Cu) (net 10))
 (segment (start 122.65 98.73) (end 126.77 98.73) (width 0.5) (layer B.Cu) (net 10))
 (segment (start 140.77 98.73) (end 141 98.5) (width 0.5) (layer B.Cu) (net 11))
 (segment (start 136.65 98.73) (end 140.77 98.73) (width 0.5) (layer B.Cu) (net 11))
 (segment (start 154.77 98.73) (end 155 98.5) (width 0.5) (layer B.Cu) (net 12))
 (segment (start 150.65 98.73) (end 154.77 98.73) (width 0.5) (layer B.Cu) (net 12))
 (segment (start 168.77 98.73) (end 169 98.5) (width 0.5) (layer B.Cu) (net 13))
 (segment (start 164.65 98.73) (end 168.77 98.73) (width 0.5) (layer B.Cu) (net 13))
 (segment (start 136.88 72.5) (end 136.65 72.73) (width 1) (layer B.Cu) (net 3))
 (segment (start 137.92 74) (end 136.65 72.73) (width 0.5) (layer B.Cu) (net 3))
 (segment (start 141.3 74) (end 137.92 74) (width 0.5) (layer B.Cu) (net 3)))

